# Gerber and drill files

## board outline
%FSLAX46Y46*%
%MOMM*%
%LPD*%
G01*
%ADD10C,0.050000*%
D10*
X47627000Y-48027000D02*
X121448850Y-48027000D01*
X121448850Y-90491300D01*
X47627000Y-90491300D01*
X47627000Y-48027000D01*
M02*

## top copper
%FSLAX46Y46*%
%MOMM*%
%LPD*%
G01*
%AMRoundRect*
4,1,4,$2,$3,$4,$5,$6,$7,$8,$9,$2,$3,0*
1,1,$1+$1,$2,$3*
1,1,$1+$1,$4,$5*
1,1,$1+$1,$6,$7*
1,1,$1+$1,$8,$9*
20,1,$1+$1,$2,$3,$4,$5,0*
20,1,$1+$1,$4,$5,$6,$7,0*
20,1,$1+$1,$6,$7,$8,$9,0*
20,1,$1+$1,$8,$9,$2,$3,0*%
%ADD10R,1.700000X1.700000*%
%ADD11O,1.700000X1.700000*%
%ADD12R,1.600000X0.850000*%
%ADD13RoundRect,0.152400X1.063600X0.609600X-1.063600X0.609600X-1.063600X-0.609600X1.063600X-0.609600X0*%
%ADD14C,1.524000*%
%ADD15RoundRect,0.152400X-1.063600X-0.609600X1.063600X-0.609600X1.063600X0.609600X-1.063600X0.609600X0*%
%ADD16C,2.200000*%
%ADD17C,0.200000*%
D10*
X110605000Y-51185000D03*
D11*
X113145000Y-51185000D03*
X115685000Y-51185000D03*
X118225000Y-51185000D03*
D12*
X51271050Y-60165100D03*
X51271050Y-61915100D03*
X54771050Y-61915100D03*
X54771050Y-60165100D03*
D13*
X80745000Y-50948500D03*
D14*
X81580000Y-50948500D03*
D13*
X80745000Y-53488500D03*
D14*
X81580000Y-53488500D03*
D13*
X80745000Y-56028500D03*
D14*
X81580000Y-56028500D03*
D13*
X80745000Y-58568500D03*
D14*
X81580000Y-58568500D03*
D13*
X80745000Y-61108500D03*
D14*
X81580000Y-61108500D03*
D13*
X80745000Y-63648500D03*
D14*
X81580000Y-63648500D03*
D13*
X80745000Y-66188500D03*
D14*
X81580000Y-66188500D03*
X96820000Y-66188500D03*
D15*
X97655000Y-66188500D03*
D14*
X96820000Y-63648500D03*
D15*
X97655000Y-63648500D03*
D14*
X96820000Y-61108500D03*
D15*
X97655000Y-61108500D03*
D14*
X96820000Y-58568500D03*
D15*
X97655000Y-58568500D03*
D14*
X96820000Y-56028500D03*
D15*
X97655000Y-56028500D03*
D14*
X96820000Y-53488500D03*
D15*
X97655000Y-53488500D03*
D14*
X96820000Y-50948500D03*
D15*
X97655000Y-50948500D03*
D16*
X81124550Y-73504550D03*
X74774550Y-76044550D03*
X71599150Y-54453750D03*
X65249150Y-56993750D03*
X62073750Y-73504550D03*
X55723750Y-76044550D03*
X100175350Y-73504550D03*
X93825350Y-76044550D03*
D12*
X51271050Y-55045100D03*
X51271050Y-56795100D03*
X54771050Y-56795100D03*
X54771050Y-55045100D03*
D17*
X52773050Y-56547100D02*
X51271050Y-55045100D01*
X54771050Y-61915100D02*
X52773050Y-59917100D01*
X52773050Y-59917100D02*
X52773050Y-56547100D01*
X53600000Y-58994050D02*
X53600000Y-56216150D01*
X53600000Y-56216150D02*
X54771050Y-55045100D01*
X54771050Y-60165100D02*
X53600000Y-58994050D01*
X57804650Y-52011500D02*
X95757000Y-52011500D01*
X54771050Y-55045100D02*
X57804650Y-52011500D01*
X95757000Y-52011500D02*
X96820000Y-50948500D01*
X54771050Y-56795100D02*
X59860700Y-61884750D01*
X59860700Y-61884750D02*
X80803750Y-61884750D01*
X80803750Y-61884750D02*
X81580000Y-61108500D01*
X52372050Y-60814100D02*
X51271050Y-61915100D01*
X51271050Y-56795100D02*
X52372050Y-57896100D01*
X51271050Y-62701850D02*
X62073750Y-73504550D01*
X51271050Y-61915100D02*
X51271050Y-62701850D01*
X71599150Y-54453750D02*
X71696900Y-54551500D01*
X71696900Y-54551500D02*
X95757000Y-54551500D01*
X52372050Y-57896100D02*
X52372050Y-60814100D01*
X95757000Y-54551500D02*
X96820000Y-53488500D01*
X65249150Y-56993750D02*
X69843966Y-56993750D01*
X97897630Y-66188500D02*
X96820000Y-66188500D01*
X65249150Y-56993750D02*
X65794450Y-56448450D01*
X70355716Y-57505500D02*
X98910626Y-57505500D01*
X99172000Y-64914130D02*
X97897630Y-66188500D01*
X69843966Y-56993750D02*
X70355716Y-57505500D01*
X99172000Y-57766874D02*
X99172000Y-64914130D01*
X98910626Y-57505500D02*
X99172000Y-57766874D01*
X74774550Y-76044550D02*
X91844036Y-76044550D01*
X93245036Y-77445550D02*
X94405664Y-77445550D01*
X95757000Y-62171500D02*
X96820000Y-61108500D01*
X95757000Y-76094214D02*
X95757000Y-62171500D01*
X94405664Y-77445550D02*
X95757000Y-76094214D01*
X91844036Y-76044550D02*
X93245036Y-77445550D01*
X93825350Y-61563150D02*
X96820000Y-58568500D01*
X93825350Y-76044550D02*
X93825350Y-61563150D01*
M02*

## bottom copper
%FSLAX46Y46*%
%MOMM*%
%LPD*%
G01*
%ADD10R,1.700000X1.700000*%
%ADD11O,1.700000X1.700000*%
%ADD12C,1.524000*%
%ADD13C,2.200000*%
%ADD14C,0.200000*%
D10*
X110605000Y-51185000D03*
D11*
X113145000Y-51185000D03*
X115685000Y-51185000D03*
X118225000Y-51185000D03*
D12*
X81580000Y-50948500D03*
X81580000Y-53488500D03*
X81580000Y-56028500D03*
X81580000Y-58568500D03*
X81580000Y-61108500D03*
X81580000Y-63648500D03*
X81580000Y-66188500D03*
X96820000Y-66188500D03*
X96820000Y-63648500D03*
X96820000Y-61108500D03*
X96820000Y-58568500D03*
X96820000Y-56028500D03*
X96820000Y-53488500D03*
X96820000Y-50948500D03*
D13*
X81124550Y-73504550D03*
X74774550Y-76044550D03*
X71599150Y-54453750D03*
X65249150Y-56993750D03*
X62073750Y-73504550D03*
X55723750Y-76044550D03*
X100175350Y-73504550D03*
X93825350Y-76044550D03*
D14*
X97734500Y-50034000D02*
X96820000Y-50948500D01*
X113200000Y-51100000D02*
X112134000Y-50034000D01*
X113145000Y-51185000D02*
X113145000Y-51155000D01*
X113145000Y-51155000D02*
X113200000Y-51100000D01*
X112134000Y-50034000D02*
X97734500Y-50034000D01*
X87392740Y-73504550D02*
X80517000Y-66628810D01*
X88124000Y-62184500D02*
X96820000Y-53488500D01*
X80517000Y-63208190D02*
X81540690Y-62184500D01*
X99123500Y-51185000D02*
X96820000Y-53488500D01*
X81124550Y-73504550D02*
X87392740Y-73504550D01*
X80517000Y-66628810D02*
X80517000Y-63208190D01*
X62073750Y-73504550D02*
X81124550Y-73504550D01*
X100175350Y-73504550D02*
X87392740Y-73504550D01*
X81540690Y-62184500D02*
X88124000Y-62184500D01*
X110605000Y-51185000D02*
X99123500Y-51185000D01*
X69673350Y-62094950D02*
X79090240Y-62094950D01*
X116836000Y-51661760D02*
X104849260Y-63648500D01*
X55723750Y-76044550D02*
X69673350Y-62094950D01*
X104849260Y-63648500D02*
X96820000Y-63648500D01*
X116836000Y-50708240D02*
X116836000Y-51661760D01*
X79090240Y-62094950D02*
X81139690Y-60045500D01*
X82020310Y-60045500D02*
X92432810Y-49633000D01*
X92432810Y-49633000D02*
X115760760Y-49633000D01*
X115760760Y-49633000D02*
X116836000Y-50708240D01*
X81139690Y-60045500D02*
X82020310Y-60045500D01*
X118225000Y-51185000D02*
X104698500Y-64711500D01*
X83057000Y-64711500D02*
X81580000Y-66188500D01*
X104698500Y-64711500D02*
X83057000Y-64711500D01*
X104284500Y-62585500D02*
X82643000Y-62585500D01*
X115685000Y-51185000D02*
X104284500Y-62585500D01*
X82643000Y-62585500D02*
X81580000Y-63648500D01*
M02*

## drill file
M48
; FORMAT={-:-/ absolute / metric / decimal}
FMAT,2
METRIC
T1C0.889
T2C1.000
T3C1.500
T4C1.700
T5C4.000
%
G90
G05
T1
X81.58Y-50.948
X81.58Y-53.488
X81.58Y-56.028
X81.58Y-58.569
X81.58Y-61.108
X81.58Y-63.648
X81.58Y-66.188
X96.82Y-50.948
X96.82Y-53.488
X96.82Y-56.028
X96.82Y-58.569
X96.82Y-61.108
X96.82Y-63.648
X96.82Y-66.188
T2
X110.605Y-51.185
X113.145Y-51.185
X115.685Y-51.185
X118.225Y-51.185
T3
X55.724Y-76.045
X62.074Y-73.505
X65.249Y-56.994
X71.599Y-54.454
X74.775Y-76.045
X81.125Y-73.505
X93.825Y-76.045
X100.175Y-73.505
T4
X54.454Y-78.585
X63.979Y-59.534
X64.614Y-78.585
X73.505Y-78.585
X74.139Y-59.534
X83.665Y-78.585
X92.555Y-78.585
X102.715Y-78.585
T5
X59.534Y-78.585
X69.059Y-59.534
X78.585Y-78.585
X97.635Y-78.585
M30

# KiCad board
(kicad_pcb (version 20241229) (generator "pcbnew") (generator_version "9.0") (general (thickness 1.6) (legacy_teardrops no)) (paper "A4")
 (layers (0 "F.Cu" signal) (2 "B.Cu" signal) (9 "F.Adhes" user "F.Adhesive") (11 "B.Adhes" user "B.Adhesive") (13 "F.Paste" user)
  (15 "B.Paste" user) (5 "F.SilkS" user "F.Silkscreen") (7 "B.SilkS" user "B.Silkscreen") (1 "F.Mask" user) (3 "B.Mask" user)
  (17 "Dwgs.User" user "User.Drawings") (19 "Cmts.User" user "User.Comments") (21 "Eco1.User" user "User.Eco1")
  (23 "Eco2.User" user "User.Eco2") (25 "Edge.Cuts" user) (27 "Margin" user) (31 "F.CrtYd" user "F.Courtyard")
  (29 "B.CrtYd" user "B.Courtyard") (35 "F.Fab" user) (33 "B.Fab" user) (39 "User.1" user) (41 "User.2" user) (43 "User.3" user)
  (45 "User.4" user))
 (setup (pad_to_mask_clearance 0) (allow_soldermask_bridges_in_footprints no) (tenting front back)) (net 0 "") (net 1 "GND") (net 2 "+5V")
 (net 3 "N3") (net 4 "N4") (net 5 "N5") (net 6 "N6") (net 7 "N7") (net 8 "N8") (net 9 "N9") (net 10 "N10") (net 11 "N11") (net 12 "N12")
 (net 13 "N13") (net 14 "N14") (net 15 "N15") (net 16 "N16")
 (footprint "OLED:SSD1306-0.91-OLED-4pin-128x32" (layer "F.Cu") (at 108.415 87.685 90)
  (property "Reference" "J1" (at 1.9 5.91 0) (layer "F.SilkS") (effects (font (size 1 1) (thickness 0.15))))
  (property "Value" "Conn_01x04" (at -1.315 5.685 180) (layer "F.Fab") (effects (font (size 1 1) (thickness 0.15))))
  (pad "1" thru_hole rect (at 36.5 2.19 90) (size 1.7 1.7) (drill 1) (layers "*.Cu" "*.Mask") (remove_unused_layers no) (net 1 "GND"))
  (pad "2" thru_hole oval (at 36.5 4.73 90) (size 1.7 1.7) (drill 1) (layers "*.Cu" "*.Mask") (remove_unused_layers no) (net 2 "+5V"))
  (pad "3" thru_hole oval (at 36.5 7.27 90) (size 1.7 1.7) (drill 1) (layers "*.Cu" "*.Mask") (remove_unused_layers no) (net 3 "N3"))
  (pad "4" thru_hole oval (at 36.5 9.81 90) (size 1.7 1.7) (drill 1) (layers "*.Cu" "*.Mask") (remove_unused_layers no) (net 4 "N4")))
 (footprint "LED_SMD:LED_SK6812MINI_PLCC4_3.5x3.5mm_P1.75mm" (layer "F.Cu") (at 53.02105 61.0401)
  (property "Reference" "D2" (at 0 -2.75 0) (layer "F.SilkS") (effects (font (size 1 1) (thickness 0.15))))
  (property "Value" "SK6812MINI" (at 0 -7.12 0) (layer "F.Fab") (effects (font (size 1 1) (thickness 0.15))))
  (pad "1" smd rect (at -1.75 -0.875) (size 1.6 0.85) (layers "F.Cu" "F.Mask" "F.Paste") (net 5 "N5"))
  (pad "2" smd rect (at -1.75 0.875) (size 1.6 0.85) (layers "F.Cu" "F.Mask" "F.Paste") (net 1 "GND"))
  (pad "3" smd rect (at 1.75 0.875) (size 1.6 0.85) (layers "F.Cu" "F.Mask" "F.Paste") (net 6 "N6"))
  (pad "4" smd rect (at 1.75 -0.875) (size 1.6 0.85) (layers "F.Cu" "F.Mask" "F.Paste") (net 2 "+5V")))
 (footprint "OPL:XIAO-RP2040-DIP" (layer "F.Cu") (at 89.2 58.5685)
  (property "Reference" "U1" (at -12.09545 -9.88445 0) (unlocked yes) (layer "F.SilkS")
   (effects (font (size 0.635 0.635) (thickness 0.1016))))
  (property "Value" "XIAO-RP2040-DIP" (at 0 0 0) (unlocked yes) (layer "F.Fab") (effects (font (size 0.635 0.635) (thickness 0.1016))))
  (pad "1" smd roundrect (at -8.455 -7.62 180) (size 2.432 1.524) (layers "F.Cu" "F.Mask") (roundrect_rratio 0.1) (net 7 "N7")
   (thermal_bridge_angle 45))
  (pad "1" thru_hole circle (at -7.62 -7.62 180) (size 1.524 1.524) (drill 0.889) (layers "*.Cu" "*.Mask") (remove_unused_layers no)
   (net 7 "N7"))
  (pad "2" smd roundrect (at -8.455 -5.08 180) (size 2.432 1.524) (layers "F.Cu" "F.Mask") (roundrect_rratio 0.1) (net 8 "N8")
   (thermal_bridge_angle 45))
  (pad "2" thru_hole circle (at -7.62 -5.08 180) (size 1.524 1.524) (drill 0.889) (layers "*.Cu" "*.Mask") (remove_unused_layers no)
   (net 8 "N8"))
  (pad "3" smd roundrect (at -8.455 -2.54 180) (size 2.432 1.524) (layers "F.Cu" "F.Mask") (roundrect_rratio 0.1) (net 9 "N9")
   (thermal_bridge_angle 45))
  (pad "3" thru_hole circle (at -7.62 -2.54 180) (size 1.524 1.524) (drill 0.889) (layers "*.Cu" "*.Mask") (remove_unused_layers no)
   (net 9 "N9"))
  (pad "4" smd roundrect (at -8.455 0 180) (size 2.432 1.524) (layers "F.Cu" "F.Mask") (roundrect_rratio 0.1) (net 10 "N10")
   (thermal_bridge_angle 45))
  (pad "4" thru_hole circle (at -7.62 0 180) (size 1.524 1.524) (drill 0.889) (layers "*.Cu" "*.Mask") (remove_unused_layers no)
   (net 10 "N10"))
  (pad "5" smd roundrect (at -8.455 2.54 180) (size 2.432 1.524) (layers "F.Cu" "F.Mask") (roundrect_rratio 0.1) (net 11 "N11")
   (thermal_bridge_angle 45))
  (pad "5" thru_hole circle (at -7.62 2.54 180) (size 1.524 1.524) (drill 0.889) (layers "*.Cu" "*.Mask") (remove_unused_layers no)
   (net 11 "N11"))
  (pad "6" smd roundrect (at -8.455 5.08 180) (size 2.432 1.524) (layers "F.Cu" "F.Mask") (roundrect_rratio 0.1) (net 3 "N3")
   (thermal_bridge_angle 45))
  (pad "6" thru_hole circle (at -7.62 5.08 180) (size 1.524 1.524) (drill 0.889) (layers "*.Cu" "*.Mask") (remove_unused_layers no)
   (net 3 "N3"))
  (pad "7" smd roundrect (at -8.455 7.62 180) (size 2.432 1.524) (layers "F.Cu" "F.Mask") (roundrect_rratio 0.1) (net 4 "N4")
   (thermal_bridge_angle 45))
  (pad "7" thru_hole circle (at -7.62 7.62 180) (size 1.524 1.524) (drill 0.889) (layers "*.Cu" "*.Mask") (remove_unused_layers no)
   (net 4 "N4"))
  (pad "8" thru_hole circle (at 7.62 7.62) (size 1.524 1.524) (drill 0.889) (layers "*.Cu" "*.Mask") (remove_unused_layers no)
   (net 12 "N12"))
  (pad "8" smd roundrect (at 8.455 7.62) (size 2.432 1.524) (layers "F.Cu" "F.Mask") (roundrect_rratio 0.1) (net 12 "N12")
   (thermal_bridge_angle 45))
  (pad "9" thru_hole circle (at 7.62 5.08) (size 1.524 1.524) (drill 0.889) (layers "*.Cu" "*.Mask") (remove_unused_layers no)
   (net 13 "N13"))
  (pad "9" smd roundrect (at 8.455 5.08) (size 2.432 1.524) (layers "F.Cu" "F.Mask") (roundrect_rratio 0.1) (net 13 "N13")
   (thermal_bridge_angle 45))
  (pad "10" thru_hole circle (at 7.62 2.54) (size 1.524 1.524) (drill 0.889) (layers "*.Cu" "*.Mask") (remove_unused_layers no)
   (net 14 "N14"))
  (pad "10" smd roundrect (at 8.455 2.54) (size 2.432 1.524) (layers "F.Cu" "F.Mask") (roundrect_rratio 0.1) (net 14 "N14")
   (thermal_bridge_angle 45))
  (pad "11" thru_hole circle (at 7.62 0) (size 1.524 1.524) (drill 0.889) (layers "*.Cu" "*.Mask") (remove_unused_layers no) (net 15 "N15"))
  (pad "11" smd roundrect (at 8.455 0) (size 2.432 1.524) (layers "F.Cu" "F.Mask") (roundrect_rratio 0.1) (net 15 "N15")
   (thermal_bridge_angle 45))
  (pad "12" thru_hole circle (at 7.62 -2.54) (size 1.524 1.524) (drill 0.889) (layers "*.Cu" "*.Mask") (remove_unused_layers no)
   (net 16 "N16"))
  (pad "12" smd roundrect (at 8.455 -2.54) (size 2.432 1.524) (layers "F.Cu" "F.Mask") (roundrect_rratio 0.1) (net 16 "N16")
   (thermal_bridge_angle 45))
  (pad "13" thru_hole circle (at 7.62 -5.08) (size 1.524 1.524) (drill 0.889) (layers "*.Cu" "*.Mask") (remove_unused_layers no)
   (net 1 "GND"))
  (pad "13" smd roundrect (at 8.455 -5.08) (size 2.432 1.524) (layers "F.Cu" "F.Mask") (roundrect_rratio 0.1) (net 1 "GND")
   (thermal_bridge_angle 45))
  (pad "14" thru_hole circle (at 7.62 -7.62) (size 1.524 1.524) (drill 0.889) (layers "*.Cu" "*.Mask") (remove_unused_layers no)
   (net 2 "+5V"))
  (pad "14" smd roundrect (at 8.455 -7.62) (size 2.432 1.524) (layers "F.Cu" "F.Mask") (roundrect_rratio 0.1) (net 2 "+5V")
   (thermal_bridge_angle 45)))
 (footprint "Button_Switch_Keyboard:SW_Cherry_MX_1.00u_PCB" (layer "F.Cu") (at 81.12455 73.50455)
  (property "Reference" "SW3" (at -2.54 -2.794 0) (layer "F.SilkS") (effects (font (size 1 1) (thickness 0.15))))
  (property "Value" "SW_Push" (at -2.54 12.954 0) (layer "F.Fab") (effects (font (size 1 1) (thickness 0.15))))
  (pad "" np_thru_hole circle (at -7.62 5.08) (size 1.7 1.7) (drill 1.7) (layers "*.Cu" "*.Mask"))
  (pad "" np_thru_hole circle (at -2.54 5.08) (size 4 4) (drill 4) (layers "*.Cu" "*.Mask"))
  (pad "" np_thru_hole circle (at 2.54 5.08) (size 1.7 1.7) (drill 1.7) (layers "*.Cu" "*.Mask"))
  (pad "1" thru_hole circle (at 0 0) (size 2.2 2.2) (drill 1.5) (layers "*.Cu" "*.Mask") (remove_unused_layers no) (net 1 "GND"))
  (pad "2" thru_hole circle (at -6.35 2.54) (size 2.2 2.2) (drill 1.5) (layers "*.Cu" "*.Mask") (remove_unused_layers no) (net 14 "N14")))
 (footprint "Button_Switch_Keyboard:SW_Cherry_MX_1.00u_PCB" (layer "F.Cu") (at 71.59915 54.45375)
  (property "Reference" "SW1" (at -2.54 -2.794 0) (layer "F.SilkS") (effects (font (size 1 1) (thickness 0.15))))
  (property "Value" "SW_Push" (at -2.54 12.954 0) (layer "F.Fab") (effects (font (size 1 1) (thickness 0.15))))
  (pad "" np_thru_hole circle (at -7.62 5.08) (size 1.7 1.7) (drill 1.7) (layers "*.Cu" "*.Mask"))
  (pad "" np_thru_hole circle (at -2.54 5.08) (size 4 4) (drill 4) (layers "*.Cu" "*.Mask"))
  (pad "" np_thru_hole circle (at 2.54 5.08) (size 1.7 1.7) (drill 1.7) (layers "*.Cu" "*.Mask"))
  (pad "1" thru_hole circle (at 0 0) (size 2.2 2.2) (drill 1.5) (layers "*.Cu" "*.Mask") (remove_unused_layers no) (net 1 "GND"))
  (pad "2" thru_hole circle (at -6.35 2.54) (size 2.2 2.2) (drill 1.5) (layers "*.Cu" "*.Mask") (remove_unused_layers no) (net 12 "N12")))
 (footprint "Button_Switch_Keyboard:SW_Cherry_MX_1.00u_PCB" (layer "F.Cu") (at 62.07375 73.50455)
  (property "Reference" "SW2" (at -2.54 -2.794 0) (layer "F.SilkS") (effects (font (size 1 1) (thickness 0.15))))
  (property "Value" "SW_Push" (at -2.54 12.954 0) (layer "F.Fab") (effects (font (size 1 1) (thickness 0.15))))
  (pad "" np_thru_hole circle (at -7.62 5.08) (size 1.7 1.7) (drill 1.7) (layers "*.Cu" "*.Mask"))
  (pad "" np_thru_hole circle (at -2.54 5.08) (size 4 4) (drill 4) (layers "*.Cu" "*.Mask"))
  (pad "" np_thru_hole circle (at 2.54 5.08) (size 1.7 1.7) (drill 1.7) (layers "*.Cu" "*.Mask"))
  (pad "1" thru_hole circle (at 0 0) (size 2.2 2.2) (drill 1.5) (layers "*.Cu" "*.Mask") (remove_unused_layers no) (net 1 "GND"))
  (pad "2" thru_hole circle (at -6.35 2.54) (size 2.2 2.2) (drill 1.5) (layers "*.Cu" "*.Mask") (remove_unused_layers no) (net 13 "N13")))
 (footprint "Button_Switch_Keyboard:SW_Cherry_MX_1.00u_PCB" (layer "F.Cu") (at 100.17535 73.50455)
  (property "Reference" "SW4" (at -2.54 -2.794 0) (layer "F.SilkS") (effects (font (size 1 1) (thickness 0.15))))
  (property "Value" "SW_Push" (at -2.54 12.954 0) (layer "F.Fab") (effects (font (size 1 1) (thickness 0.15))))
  (pad "" np_thru_hole circle (at -7.62 5.08) (size 1.7 1.7) (drill 1.7) (layers "*.Cu" "*.Mask"))
  (pad "" np_thru_hole circle (at -2.54 5.08) (size 4 4) (drill 4) (layers "*.Cu" "*.Mask"))
  (pad "" np_thru_hole circle (at 2.54 5.08) (size 1.7 1.7) (drill 1.7) (layers "*.Cu" "*.Mask"))
  (pad "1" thru_hole circle (at 0 0) (size 2.2 2.2) (drill 1.5) (layers "*.Cu" "*.Mask") (remove_unused_layers no) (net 1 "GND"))
  (pad "2" thru_hole circle (at -6.35 2.54) (size 2.2 2.2) (drill 1.5) (layers "*.Cu" "*.Mask") (remove_unused_layers no) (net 15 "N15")))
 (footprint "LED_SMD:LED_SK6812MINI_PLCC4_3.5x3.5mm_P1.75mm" (layer "F.Cu") (at 53.02105 55.9201)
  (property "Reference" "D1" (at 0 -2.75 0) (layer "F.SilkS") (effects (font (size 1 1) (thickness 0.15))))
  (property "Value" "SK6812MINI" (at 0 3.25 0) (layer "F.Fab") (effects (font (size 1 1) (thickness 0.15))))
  (pad "1" smd rect (at -1.75 -0.875) (size 1.6 0.85) (layers "F.Cu" "F.Mask" "F.Paste") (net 6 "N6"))
  (pad "2" smd rect (at -1.75 0.875) (size 1.6 0.85) (layers "F.Cu" "F.Mask" "F.Paste") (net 1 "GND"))
  (pad "3" smd rect (at 1.75 0.875) (size 1.6 0.85) (layers "F.Cu" "F.Mask" "F.Paste") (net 11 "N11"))
  (pad "4" smd rect (at 1.75 -0.875) (size 1.6 0.85) (layers "F.Cu" "F.Mask" "F.Paste") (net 2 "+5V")))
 (gr_rect (start 47.627 48.027) (end 121.44885 90.4913) (stroke (width 0.05) (type default)) (fill no) (layer "Edge.Cuts"))
 (segment (start 52.77305 56.5471) (end 51.27105 55.0451) (width 0.2) (layer "F.Cu") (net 6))
 (segment (start 54.77105 61.9151) (end 52.77305 59.9171) (width 0.2) (layer "F.Cu") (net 6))
 (segment (start 52.77305 59.9171) (end 52.77305 56.5471) (width 0.2) (layer "F.Cu") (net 6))
 (segment (start 53.6 58.99405) (end 53.6 56.21615) (width 0.2) (layer "F.Cu") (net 2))
 (segment (start 53.6 56.21615) (end 54.77105 55.0451) (width 0.2) (layer "F.Cu") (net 2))
 (segment (start 54.77105 60.1651) (end 53.6 58.99405) (width 0.2) (layer "F.Cu") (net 2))
 (segment (start 57.80465 52.0115) (end 95.757 52.0115) (width 0.2) (layer "F.Cu") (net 2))
 (segment (start 54.77105 55.0451) (end 57.80465 52.0115) (width 0.2) (layer "F.Cu") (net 2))
 (segment (start 95.757 52.0115) (end 96.82 50.9485) (width 0.2) (layer "F.Cu") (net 2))
 (segment (start 97.7345 50.034) (end 96.82 50.9485) (width 0.2) (layer "B.Cu") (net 2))
 (segment (start 113.2 51.1) (end 112.134 50.034) (width 0.2) (layer "B.Cu") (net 2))
 (segment (start 113.145 51.185) (end 113.145 51.155) (width 0.2) (layer "B.Cu") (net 2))
 (segment (start 113.145 51.155) (end 113.2 51.1) (width 0.2) (layer "B.Cu") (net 2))
 (segment (start 112.134 50.034) (end 97.7345 50.034) (width 0.2) (layer "B.Cu") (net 2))
 (segment (start 54.77105 56.7951) (end 59.8607 61.88475) (width 0.2) (layer "F.Cu") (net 11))
 (segment (start 59.8607 61.88475) (end 80.80375 61.88475) (width 0.2) (layer "F.Cu") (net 11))
 (segment (start 80.80375 61.88475) (end 81.58 61.1085) (width 0.2) (layer "F.Cu") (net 11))
 (segment (start 52.37205 60.8141) (end 51.27105 61.9151) (width 0.2) (layer "F.Cu") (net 1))
 (segment (start 51.27105 56.7951) (end 52.37205 57.8961) (width 0.2) (layer "F.Cu") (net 1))
 (segment (start 51.27105 62.70185) (end 62.07375 73.50455) (width 0.2) (layer "F.Cu") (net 1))
 (segment (start 51.27105 61.9151) (end 51.27105 62.70185) (width 0.2) (layer "F.Cu") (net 1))
 (segment (start 71.59915 54.45375) (end 71.6969 54.5515) (width 0.2) (layer "F.Cu") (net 1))
 (segment (start 71.6969 54.5515) (end 95.757 54.5515) (width 0.2) (layer "F.Cu") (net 1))
 (segment (start 52.37205 57.8961) (end 52.37205 60.8141) (width 0.2) (layer "F.Cu") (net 1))
 (segment (start 95.757 54.5515) (end 96.82 53.4885) (width 0.2) (layer "F.Cu") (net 1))
 (segment (start 87.39274 73.50455) (end 80.517 66.62881) (width 0.2) (layer "B.Cu") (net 1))
 (segment (start 88.124 62.1845) (end 96.82 53.4885) (width 0.2) (layer "B.Cu") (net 1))
 (segment (start 80.517 63.20819) (end 81.54069 62.1845) (width 0.2) (layer "B.Cu") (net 1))
 (segment (start 99.1235 51.185) (end 96.82 53.4885) (width 0.2) (layer "B.Cu") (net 1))
 (segment (start 81.12455 73.50455) (end 87.39274 73.50455) (width 0.2) (layer "B.Cu") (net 1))
 (segment (start 80.517 66.62881) (end 80.517 63.20819) (width 0.2) (layer "B.Cu") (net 1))
 (segment (start 62.07375 73.50455) (end 81.12455 73.50455) (width 0.2) (layer "B.Cu") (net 1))
 (segment (start 100.17535 73.50455) (end 87.39274 73.50455) (width 0.2) (layer "B.Cu") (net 1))
 (segment (start 81.54069 62.1845) (end 88.124 62.1845) (width 0.2) (layer "B.Cu") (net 1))
 (segment (start 110.605 51.185) (end 99.1235 51.185) (width 0.2) (layer "B.Cu") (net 1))
 (segment (start 65.24915 56.99375) (end 69.843966 56.99375) (width 0.2) (layer "F.Cu") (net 12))
 (segment (start 97.89763 66.1885) (end 96.82 66.1885) (width 0.2) (layer "F.Cu") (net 12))
 (segment (start 65.24915 56.99375) (end 65.79445 56.44845) (width 0.2) (layer "F.Cu") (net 12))
 (segment (start 70.355716 57.5055) (end 98.910626 57.5055) (width 0.2) (layer "F.Cu") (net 12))
 (segment (start 99.172 64.91413) (end 97.89763 66.1885) (width 0.2) (layer "F.Cu") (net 12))
 (segment (start 69.843966 56.99375) (end 70.355716 57.5055) (width 0.2) (layer "F.Cu") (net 12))
 (segment (start 99.172 57.766874) (end 99.172 64.91413) (width 0.2) (layer "F.Cu") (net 12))
 (segment (start 98.910626 57.5055) (end 99.172 57.766874) (width 0.2) (layer "F.Cu") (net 12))
 (segment (start 69.67335 62.09495) (end 79.09024 62.09495) (width 0.2) (layer "B.Cu") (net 13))
 (segment (start 116.836 51.66176) (end 104.84926 63.6485) (width 0.2) (layer "B.Cu") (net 13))
 (segment (start 55.72375 76.04455) (end 69.67335 62.09495) (width 0.2) (layer "B.Cu") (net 13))
 (segment (start 104.84926 63.6485) (end 96.82 63.6485) (width 0.2) (layer "B.Cu") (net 13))
 (segment (start 116.836 50.70824) (end 116.836 51.66176) (width 0.2) (layer "B.Cu") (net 13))
 (segment (start 79.09024 62.09495) (end 81.13969 60.0455) (width 0.2) (layer "B.Cu") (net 13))
 (segment (start 82.02031 60.0455) (end 92.43281 49.633) (width 0.2) (layer "B.Cu") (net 13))
 (segment (start 92.43281 49.633) (end 115.76076 49.633) (width 0.2) (layer "B.Cu") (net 13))
 (segment (start 115.76076 49.633) (end 116.836 50.70824) (width 0.2) (layer "B.Cu") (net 13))
 (segment (start 81.13969 60.0455) (end 82.02031 60.0455) (width 0.2) (layer "B.Cu") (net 13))
 (segment (start 74.77455 76.04455) (end 91.844036 76.04455) (width 0.2) (layer "F.Cu") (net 14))
 (segment (start 93.245036 77.44555) (end 94.405664 77.44555) (width 0.2) (layer "F.Cu") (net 14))
 (segment (start 95.757 62.1715) (end 96.82 61.1085) (width 0.2) (layer "F.Cu") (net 14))
 (segment (start 95.757 76.094214) (end 95.757 62.1715) (width 0.2) (layer "F.Cu") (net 14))
 (segment (start 94.405664 77.44555) (end 95.757 76.094214) (width 0.2) (layer "F.Cu") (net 14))
 (segment (start 91.844036 76.04455) (end 93.245036 77.44555) (width 0.2) (layer "F.Cu") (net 14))
 (segment (start 93.82535 61.56315) (end 96.82 58.5685) (width 0.2) (layer "F.Cu") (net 15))
 (segment (start 93.82535 76.04455) (end 93.82535 61.56315) (width 0.2) (layer "F.Cu") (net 15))
 (segment (start 118.225 51.185) (end 104.6985 64.7115) (width 0.2) (layer "B.Cu") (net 4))
 (segment (start 83.057 64.7115) (end 81.58 66.1885) (width 0.2) (layer "B.Cu") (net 4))
 (segment (start 104.6985 64.7115) (end 83.057 64.7115) (width 0.2) (layer "B.Cu") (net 4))
 (segment (start 104.2845 62.5855) (end 82.643 62.5855) (width 0.2) (layer "B.Cu") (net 3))
 (segment (start 115.685 51.185) (end 104.2845 62.5855) (width 0.2) (layer "B.Cu") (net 3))
 (segment (start 82.643 62.5855) (end 81.58 63.6485) (width 0.2) (layer "B.Cu") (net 3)))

